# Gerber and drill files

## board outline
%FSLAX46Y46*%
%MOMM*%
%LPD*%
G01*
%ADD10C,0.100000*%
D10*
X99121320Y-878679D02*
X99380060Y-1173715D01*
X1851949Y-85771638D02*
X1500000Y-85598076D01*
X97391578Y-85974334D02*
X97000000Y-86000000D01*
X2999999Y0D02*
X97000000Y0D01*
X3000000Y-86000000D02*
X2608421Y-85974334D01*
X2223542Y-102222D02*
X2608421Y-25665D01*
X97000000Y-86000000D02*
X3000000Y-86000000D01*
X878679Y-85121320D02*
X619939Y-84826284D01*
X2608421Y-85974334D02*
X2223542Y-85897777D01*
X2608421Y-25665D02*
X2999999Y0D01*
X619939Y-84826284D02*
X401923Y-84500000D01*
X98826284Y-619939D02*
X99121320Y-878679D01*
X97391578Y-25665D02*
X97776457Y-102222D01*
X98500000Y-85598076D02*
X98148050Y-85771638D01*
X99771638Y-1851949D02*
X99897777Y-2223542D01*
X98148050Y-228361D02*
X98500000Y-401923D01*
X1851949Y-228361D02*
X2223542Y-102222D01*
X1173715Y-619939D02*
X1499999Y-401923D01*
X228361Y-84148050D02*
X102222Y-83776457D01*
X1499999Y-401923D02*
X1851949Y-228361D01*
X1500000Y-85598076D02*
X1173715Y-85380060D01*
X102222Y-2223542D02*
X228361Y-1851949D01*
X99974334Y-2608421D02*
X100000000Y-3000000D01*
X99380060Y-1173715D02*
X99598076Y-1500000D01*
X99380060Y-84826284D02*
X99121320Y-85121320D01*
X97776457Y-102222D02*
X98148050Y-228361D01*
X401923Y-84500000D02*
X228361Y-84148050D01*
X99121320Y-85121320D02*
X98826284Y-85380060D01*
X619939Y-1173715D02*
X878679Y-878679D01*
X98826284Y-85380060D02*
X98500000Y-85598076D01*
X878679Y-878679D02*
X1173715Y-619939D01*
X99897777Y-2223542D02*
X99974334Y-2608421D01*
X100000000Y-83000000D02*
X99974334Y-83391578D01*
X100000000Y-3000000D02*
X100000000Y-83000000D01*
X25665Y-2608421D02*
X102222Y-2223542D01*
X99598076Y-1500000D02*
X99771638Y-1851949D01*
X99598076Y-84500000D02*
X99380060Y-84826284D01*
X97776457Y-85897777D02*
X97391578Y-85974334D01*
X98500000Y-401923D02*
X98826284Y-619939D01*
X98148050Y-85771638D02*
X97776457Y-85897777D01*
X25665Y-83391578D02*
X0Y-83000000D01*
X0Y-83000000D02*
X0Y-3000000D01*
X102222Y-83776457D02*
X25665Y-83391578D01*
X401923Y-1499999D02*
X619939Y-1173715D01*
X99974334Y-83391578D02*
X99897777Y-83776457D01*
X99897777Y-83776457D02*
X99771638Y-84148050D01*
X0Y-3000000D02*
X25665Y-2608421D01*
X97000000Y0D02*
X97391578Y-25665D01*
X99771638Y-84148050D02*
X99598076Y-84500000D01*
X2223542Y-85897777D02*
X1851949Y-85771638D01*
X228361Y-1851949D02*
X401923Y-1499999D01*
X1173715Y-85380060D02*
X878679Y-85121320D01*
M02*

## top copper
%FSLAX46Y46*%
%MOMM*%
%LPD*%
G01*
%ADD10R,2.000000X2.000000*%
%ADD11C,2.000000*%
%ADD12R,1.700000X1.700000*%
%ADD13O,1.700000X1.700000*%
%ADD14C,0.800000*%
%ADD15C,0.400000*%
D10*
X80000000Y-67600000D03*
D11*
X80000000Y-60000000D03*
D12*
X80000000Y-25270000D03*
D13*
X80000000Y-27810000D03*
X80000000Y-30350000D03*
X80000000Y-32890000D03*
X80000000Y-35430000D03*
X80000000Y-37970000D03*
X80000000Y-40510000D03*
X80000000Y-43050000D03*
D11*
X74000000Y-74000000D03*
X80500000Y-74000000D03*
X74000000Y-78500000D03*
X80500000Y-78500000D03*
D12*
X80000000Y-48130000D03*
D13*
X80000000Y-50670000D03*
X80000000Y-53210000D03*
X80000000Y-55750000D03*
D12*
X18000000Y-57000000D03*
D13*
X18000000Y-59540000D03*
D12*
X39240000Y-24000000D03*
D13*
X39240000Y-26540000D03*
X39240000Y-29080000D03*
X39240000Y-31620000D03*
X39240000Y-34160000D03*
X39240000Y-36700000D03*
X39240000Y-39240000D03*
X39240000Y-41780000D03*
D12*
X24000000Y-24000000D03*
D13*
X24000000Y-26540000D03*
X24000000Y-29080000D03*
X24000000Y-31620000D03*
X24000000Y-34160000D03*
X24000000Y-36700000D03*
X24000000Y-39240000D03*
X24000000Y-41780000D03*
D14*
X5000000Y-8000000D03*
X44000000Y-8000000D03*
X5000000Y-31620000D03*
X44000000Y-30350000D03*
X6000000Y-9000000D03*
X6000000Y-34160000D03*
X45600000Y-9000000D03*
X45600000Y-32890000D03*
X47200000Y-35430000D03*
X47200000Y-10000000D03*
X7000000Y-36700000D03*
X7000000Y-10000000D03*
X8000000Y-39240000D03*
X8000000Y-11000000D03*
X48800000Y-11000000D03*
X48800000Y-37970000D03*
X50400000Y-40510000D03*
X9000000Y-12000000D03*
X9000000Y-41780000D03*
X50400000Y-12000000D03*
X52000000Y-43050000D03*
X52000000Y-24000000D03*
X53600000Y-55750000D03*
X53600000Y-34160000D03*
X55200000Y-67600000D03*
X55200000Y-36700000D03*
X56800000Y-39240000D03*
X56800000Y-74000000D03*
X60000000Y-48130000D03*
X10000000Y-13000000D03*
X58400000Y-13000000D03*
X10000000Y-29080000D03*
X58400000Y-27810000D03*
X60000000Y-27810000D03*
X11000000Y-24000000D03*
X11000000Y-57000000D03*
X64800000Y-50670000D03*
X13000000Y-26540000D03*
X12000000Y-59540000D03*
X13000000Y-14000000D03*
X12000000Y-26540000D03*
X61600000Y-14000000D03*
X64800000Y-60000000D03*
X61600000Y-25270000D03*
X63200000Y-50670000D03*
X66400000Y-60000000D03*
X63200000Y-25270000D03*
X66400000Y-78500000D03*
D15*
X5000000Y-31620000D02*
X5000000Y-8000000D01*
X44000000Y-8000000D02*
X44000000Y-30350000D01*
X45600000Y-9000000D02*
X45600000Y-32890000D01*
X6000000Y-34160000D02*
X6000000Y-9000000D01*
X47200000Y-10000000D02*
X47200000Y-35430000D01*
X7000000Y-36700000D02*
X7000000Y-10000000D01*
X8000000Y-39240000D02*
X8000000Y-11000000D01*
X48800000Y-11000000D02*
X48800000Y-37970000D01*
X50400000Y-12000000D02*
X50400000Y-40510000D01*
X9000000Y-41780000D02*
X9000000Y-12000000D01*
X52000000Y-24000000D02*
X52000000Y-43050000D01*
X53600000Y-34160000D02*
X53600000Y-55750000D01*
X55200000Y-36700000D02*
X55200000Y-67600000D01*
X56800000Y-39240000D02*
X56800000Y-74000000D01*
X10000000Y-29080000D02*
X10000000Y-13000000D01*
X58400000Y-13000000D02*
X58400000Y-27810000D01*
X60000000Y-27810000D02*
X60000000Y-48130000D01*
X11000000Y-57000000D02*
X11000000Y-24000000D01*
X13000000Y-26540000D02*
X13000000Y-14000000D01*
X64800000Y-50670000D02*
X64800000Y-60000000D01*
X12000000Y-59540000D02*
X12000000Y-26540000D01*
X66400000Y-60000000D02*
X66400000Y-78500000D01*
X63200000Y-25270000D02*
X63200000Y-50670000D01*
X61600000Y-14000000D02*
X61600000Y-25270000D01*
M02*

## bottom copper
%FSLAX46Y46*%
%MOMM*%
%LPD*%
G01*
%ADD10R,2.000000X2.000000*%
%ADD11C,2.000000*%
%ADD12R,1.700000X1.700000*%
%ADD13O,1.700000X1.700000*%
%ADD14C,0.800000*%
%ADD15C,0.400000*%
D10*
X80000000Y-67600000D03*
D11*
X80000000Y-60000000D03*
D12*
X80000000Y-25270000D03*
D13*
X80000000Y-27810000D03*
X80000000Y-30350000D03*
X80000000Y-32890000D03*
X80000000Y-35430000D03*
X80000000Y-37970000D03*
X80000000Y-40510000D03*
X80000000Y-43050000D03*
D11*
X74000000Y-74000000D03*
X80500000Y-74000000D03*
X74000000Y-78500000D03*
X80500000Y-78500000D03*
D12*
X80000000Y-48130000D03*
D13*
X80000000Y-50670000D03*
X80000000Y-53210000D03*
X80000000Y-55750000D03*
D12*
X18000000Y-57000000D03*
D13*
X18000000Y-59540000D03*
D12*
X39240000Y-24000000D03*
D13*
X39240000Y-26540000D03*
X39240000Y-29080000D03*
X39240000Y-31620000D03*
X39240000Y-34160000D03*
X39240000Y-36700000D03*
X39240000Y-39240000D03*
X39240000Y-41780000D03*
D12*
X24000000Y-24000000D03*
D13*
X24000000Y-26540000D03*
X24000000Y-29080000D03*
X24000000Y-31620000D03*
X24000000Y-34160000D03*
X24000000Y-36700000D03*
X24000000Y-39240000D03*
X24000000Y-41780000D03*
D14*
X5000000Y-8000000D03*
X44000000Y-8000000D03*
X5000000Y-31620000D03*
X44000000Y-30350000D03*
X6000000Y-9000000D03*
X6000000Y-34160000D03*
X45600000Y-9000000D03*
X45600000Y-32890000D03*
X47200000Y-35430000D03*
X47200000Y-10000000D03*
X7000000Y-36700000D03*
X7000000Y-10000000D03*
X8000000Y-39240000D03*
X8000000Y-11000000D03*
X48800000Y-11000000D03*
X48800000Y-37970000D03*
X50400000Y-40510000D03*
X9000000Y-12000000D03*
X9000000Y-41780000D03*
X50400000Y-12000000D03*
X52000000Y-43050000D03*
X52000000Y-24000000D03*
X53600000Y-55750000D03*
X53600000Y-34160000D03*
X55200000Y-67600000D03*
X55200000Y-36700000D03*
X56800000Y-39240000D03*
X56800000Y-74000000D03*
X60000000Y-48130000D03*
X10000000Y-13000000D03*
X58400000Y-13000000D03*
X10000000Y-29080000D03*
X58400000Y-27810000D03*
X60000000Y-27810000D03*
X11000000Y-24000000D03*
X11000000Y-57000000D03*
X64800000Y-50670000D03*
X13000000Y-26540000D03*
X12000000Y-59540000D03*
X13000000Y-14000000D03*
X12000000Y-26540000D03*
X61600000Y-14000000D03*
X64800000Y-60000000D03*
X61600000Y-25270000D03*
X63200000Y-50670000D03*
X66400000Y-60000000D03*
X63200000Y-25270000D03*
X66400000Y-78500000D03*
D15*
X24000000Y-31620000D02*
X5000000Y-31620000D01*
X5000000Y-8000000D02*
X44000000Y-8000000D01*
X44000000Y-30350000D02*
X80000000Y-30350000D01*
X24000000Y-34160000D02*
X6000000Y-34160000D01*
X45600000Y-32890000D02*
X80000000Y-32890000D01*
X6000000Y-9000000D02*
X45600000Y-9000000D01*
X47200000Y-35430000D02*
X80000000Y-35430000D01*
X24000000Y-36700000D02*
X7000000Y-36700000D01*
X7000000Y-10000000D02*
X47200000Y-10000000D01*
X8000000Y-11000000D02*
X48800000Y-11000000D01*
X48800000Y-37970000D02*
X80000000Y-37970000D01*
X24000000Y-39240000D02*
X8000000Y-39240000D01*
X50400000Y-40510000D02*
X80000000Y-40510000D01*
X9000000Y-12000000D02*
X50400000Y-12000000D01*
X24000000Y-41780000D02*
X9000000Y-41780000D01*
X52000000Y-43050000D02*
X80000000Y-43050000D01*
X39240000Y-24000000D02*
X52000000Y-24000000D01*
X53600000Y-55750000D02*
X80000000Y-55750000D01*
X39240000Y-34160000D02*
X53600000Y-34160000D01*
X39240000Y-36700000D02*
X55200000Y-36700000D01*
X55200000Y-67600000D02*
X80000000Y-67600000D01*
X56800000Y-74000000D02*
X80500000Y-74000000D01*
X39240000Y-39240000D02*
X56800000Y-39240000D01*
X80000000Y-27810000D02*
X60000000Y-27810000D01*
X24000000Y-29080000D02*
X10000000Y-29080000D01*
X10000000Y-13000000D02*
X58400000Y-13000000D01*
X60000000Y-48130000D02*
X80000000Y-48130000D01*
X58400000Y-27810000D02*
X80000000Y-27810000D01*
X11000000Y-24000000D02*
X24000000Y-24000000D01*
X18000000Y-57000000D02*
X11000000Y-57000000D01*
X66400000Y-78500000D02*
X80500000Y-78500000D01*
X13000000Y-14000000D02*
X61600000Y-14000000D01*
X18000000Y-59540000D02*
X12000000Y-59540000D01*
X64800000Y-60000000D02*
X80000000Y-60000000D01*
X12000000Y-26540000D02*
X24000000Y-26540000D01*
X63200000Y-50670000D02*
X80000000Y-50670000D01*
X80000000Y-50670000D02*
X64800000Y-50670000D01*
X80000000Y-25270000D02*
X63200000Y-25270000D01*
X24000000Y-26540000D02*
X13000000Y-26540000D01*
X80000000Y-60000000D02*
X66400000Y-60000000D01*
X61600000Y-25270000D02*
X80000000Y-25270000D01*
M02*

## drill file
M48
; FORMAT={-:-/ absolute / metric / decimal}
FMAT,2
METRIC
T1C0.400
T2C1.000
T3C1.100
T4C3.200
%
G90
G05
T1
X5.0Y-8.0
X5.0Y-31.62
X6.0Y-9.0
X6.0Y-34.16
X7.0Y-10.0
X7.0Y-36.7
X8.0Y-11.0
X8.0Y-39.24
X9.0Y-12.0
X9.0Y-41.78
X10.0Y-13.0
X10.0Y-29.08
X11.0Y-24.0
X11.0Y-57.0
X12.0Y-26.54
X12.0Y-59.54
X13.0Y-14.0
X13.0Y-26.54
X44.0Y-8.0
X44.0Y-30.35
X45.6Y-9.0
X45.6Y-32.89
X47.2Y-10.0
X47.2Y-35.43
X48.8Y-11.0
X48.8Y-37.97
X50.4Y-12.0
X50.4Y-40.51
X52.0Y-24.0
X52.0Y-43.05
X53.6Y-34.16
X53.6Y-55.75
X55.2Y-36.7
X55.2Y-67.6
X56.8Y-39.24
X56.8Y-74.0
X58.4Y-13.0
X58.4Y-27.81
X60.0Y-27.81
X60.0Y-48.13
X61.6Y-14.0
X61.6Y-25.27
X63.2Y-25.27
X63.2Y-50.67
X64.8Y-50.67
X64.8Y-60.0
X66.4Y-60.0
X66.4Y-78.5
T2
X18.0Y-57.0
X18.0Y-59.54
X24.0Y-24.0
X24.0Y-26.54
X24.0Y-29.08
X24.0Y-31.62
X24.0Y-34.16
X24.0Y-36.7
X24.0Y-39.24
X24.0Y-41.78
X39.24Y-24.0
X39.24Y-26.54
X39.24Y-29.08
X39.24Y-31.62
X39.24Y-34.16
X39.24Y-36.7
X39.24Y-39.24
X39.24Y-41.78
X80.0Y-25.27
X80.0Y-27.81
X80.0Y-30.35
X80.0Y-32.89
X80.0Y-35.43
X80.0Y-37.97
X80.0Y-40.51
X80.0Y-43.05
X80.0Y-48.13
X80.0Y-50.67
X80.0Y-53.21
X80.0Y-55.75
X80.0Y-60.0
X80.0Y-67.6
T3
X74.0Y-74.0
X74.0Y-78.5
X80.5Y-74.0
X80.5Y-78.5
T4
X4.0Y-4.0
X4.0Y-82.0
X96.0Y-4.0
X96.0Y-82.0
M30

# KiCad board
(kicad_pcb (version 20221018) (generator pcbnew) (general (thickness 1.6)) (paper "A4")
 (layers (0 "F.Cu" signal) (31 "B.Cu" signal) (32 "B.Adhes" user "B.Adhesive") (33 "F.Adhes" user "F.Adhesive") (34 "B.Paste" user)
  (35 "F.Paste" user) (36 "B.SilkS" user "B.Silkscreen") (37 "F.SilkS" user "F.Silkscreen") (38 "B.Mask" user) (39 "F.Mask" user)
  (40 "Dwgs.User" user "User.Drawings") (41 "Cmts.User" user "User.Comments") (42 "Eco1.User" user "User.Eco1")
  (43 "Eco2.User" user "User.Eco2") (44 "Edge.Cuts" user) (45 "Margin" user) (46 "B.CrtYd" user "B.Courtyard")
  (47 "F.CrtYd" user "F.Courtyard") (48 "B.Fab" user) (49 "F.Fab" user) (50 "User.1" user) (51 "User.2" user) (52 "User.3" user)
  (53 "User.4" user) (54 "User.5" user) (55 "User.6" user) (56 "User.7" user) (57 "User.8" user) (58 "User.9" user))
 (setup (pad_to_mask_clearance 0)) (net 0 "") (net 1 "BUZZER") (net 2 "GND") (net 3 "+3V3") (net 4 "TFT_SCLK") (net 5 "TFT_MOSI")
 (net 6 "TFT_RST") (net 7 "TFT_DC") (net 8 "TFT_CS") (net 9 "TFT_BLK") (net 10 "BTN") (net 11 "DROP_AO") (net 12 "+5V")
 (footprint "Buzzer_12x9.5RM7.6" (layer "F.Cu") (at 80 67.6 90)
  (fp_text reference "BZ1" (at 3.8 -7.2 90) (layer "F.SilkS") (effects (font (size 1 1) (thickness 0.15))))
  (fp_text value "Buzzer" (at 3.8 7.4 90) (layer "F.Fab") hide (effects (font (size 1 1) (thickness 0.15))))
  (pad "1" thru_hole rect (at 0 0 90) (size 2 2) (drill 1) (layers "*.Cu" "*.Mask") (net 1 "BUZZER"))
  (pad "2" thru_hole circle (at 7.6 0 90) (size 2 2) (drill 1) (layers "*.Cu" "*.Mask") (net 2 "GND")))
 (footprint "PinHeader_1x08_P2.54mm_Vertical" (layer "F.Cu") (at 80 25.27)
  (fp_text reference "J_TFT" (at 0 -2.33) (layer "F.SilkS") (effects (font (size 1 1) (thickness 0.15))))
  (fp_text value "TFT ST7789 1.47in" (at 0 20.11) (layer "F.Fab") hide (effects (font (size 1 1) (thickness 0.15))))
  (pad "1" thru_hole rect (at 0 0) (size 1.7 1.7) (drill 1) (layers "*.Cu" "*.Mask") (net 2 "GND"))
  (pad "2" thru_hole oval (at 0 2.54) (size 1.7 1.7) (drill 1) (layers "*.Cu" "*.Mask") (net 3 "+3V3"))
  (pad "3" thru_hole oval (at 0 5.08) (size 1.7 1.7) (drill 1) (layers "*.Cu" "*.Mask") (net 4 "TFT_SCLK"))
  (pad "4" thru_hole oval (at 0 7.62) (size 1.7 1.7) (drill 1) (layers "*.Cu" "*.Mask") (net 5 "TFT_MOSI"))
  (pad "5" thru_hole oval (at 0 10.16) (size 1.7 1.7) (drill 1) (layers "*.Cu" "*.Mask") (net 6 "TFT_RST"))
  (pad "6" thru_hole oval (at 0 12.7) (size 1.7 1.7) (drill 1) (layers "*.Cu" "*.Mask") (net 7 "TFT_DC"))
  (pad "7" thru_hole oval (at 0 15.24) (size 1.7 1.7) (drill 1) (layers "*.Cu" "*.Mask") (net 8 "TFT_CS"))
  (pad "8" thru_hole oval (at 0 17.78) (size 1.7 1.7) (drill 1) (layers "*.Cu" "*.Mask") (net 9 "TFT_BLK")))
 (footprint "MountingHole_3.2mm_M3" (layer "F.Cu") (at 4 4)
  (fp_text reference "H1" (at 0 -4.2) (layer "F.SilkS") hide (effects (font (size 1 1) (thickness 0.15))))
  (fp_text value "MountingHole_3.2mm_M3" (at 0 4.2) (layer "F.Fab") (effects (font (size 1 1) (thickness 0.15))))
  (pad "" np_thru_hole circle (at 0 0) (size 3.2 3.2) (drill 3.2) (layers "*.Cu" "*.Mask")))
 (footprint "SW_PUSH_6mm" (layer "F.Cu") (at 74 74)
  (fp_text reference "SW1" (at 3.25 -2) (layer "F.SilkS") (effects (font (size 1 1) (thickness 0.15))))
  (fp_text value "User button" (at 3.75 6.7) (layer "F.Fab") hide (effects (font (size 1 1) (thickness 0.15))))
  (pad "1" thru_hole circle (at 0 0 90) (size 2 2) (drill 1.1) (layers "*.Cu" "*.Mask") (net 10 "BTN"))
  (pad "1" thru_hole circle (at 6.5 0 90) (size 2 2) (drill 1.1) (layers "*.Cu" "*.Mask") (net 10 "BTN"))
  (pad "2" thru_hole circle (at 0 4.5 90) (size 2 2) (drill 1.1) (layers "*.Cu" "*.Mask") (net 2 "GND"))
  (pad "2" thru_hole circle (at 6.5 4.5 90) (size 2 2) (drill 1.1) (layers "*.Cu" "*.Mask") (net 2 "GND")))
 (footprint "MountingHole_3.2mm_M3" (layer "F.Cu") (at 96 82)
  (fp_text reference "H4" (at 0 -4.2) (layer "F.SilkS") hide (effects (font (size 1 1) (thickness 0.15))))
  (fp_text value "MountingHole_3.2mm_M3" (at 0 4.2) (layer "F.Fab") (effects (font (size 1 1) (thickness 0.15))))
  (pad "" np_thru_hole circle (at 0 0) (size 3.2 3.2) (drill 3.2) (layers "*.Cu" "*.Mask")))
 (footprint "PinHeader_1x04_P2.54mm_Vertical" (layer "F.Cu") (at 80 48.13)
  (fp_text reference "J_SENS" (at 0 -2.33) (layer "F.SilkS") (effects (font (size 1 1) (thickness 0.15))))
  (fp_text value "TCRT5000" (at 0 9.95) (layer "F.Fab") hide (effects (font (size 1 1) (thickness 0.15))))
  (pad "1" thru_hole rect (at 0 0) (size 1.7 1.7) (drill 1) (layers "*.Cu" "*.Mask") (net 3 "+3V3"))
  (pad "2" thru_hole oval (at 0 2.54) (size 1.7 1.7) (drill 1) (layers "*.Cu" "*.Mask") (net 2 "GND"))
  (pad "3" thru_hole oval (at 0 5.08) (size 1.7 1.7) (drill 1) (layers "*.Cu" "*.Mask"))
  (pad "4" thru_hole oval (at 0 7.62) (size 1.7 1.7) (drill 1) (layers "*.Cu" "*.Mask") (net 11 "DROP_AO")))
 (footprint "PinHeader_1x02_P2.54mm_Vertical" (layer "F.Cu") (at 18 57)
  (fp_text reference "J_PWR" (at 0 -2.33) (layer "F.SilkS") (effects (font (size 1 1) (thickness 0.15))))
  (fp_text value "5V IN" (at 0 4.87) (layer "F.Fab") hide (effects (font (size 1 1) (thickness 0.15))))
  (pad "1" thru_hole rect (at 0 0) (size 1.7 1.7) (drill 1) (layers "*.Cu" "*.Mask") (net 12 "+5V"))
  (pad "2" thru_hole oval (at 0 2.54) (size 1.7 1.7) (drill 1) (layers "*.Cu" "*.Mask") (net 2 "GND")))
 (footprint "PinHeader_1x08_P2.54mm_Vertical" (layer "F.Cu") (at 39.24 24)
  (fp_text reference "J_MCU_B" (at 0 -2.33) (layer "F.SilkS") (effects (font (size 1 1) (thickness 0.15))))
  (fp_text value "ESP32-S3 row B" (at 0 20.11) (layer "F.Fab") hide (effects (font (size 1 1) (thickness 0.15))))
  (pad "1" thru_hole rect (at 0 0) (size 1.7 1.7) (drill 1) (layers "*.Cu" "*.Mask") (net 9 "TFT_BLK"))
  (pad "2" thru_hole oval (at 0 2.54) (size 1.7 1.7) (drill 1) (layers "*.Cu" "*.Mask"))
  (pad "3" thru_hole oval (at 0 5.08) (size 1.7 1.7) (drill 1) (layers "*.Cu" "*.Mask"))
  (pad "4" thru_hole oval (at 0 7.62) (size 1.7 1.7) (drill 1) (layers "*.Cu" "*.Mask"))
  (pad "5" thru_hole oval (at 0 10.16) (size 1.7 1.7) (drill 1) (layers "*.Cu" "*.Mask") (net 11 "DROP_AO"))
  (pad "6" thru_hole oval (at 0 12.7) (size 1.7 1.7) (drill 1) (layers "*.Cu" "*.Mask") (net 1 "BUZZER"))
  (pad "7" thru_hole oval (at 0 15.24) (size 1.7 1.7) (drill 1) (layers "*.Cu" "*.Mask") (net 10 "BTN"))
  (pad "8" thru_hole oval (at 0 17.78) (size 1.7 1.7) (drill 1) (layers "*.Cu" "*.Mask")))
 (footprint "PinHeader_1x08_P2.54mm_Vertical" (layer "F.Cu") (at 24 24)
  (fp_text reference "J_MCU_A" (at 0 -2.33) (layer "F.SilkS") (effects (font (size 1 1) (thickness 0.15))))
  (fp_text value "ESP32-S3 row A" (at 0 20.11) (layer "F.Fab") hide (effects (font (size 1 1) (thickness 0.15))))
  (pad "1" thru_hole rect (at 0 0) (size 1.7 1.7) (drill 1) (layers "*.Cu" "*.Mask") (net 12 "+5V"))
  (pad "2" thru_hole oval (at 0 2.54) (size 1.7 1.7) (drill 1) (layers "*.Cu" "*.Mask") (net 2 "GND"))
  (pad "3" thru_hole oval (at 0 5.08) (size 1.7 1.7) (drill 1) (layers "*.Cu" "*.Mask") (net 3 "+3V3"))
  (pad "4" thru_hole oval (at 0 7.62) (size 1.7 1.7) (drill 1) (layers "*.Cu" "*.Mask") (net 4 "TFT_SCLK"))
  (pad "5" thru_hole oval (at 0 10.16) (size 1.7 1.7) (drill 1) (layers "*.Cu" "*.Mask") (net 5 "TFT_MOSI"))
  (pad "6" thru_hole oval (at 0 12.7) (size 1.7 1.7) (drill 1) (layers "*.Cu" "*.Mask") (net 6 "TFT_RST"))
  (pad "7" thru_hole oval (at 0 15.24) (size 1.7 1.7) (drill 1) (layers "*.Cu" "*.Mask") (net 7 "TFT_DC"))
  (pad "8" thru_hole oval (at 0 17.78) (size 1.7 1.7) (drill 1) (layers "*.Cu" "*.Mask") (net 8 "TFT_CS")))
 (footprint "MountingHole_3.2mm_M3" (layer "F.Cu") (at 4 82)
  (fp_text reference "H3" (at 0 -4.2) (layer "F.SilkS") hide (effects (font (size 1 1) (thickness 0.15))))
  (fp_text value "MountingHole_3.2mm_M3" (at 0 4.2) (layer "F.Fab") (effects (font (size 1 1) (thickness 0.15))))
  (pad "" np_thru_hole circle (at 0 0) (size 3.2 3.2) (drill 3.2) (layers "*.Cu" "*.Mask")))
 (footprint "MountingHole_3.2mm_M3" (layer "F.Cu") (at 96 4)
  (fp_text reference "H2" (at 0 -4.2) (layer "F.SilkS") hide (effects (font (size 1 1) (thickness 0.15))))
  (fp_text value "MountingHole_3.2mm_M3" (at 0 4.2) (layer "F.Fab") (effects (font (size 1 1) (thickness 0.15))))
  (pad "" np_thru_hole circle (at 0 0) (size 3.2 3.2) (drill 3.2) (layers "*.Cu" "*.Mask")))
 (gr_line (start 99.12132 0.878679) (end 99.38006 1.173715) (stroke (width 0.1) (type default)) (layer "Edge.Cuts"))
 (gr_line (start 1.851949 85.771638) (end 1.5 85.598076) (stroke (width 0.1) (type default)) (layer "Edge.Cuts"))
 (gr_line (start 97.391578 85.974334) (end 97 86) (stroke (width 0.1) (type default)) (layer "Edge.Cuts"))
 (gr_line (start 2.999999 0) (end 97 0) (stroke (width 0.1) (type default)) (layer "Edge.Cuts"))
 (gr_line (start 3 86) (end 2.608421 85.974334) (stroke (width 0.1) (type default)) (layer "Edge.Cuts"))
 (gr_line (start 2.223542 0.102222) (end 2.608421 0.025665) (stroke (width 0.1) (type default)) (layer "Edge.Cuts"))
 (gr_line (start 97 86) (end 3 86) (stroke (width 0.1) (type default)) (layer "Edge.Cuts"))
 (gr_line (start 0.878679 85.12132) (end 0.619939 84.826284) (stroke (width 0.1) (type default)) (layer "Edge.Cuts"))
 (gr_line (start 2.608421 85.974334) (end 2.223542 85.897777) (stroke (width 0.1) (type default)) (layer "Edge.Cuts"))
 (gr_line (start 2.608421 0.025665) (end 2.999999 0) (stroke (width 0.1) (type default)) (layer "Edge.Cuts"))
 (gr_line (start 0.619939 84.826284) (end 0.401923 84.5) (stroke (width 0.1) (type default)) (layer "Edge.Cuts"))
 (gr_line (start 98.826284 0.619939) (end 99.12132 0.878679) (stroke (width 0.1) (type default)) (layer "Edge.Cuts"))
 (gr_line (start 97.391578 0.025665) (end 97.776457 0.102222) (stroke (width 0.1) (type default)) (layer "Edge.Cuts"))
 (gr_line (start 98.5 85.598076) (end 98.14805 85.771638) (stroke (width 0.1) (type default)) (layer "Edge.Cuts"))
 (gr_line (start 99.771638 1.851949) (end 99.897777 2.223542) (stroke (width 0.1) (type default)) (layer "Edge.Cuts"))
 (gr_line (start 98.14805 0.228361) (end 98.5 0.401923) (stroke (width 0.1) (type default)) (layer "Edge.Cuts"))
 (gr_line (start 1.851949 0.228361) (end 2.223542 0.102222) (stroke (width 0.1) (type default)) (layer "Edge.Cuts"))
 (gr_line (start 1.173715 0.619939) (end 1.499999 0.401923) (stroke (width 0.1) (type default)) (layer "Edge.Cuts"))
 (gr_line (start 0.228361 84.14805) (end 0.102222 83.776457) (stroke (width 0.1) (type default)) (layer "Edge.Cuts"))
 (gr_line (start 1.499999 0.401923) (end 1.851949 0.228361) (stroke (width 0.1) (type default)) (layer "Edge.Cuts"))
 (gr_line (start 1.5 85.598076) (end 1.173715 85.38006) (stroke (width 0.1) (type default)) (layer "Edge.Cuts"))
 (gr_line (start 0.102222 2.223542) (end 0.228361 1.851949) (stroke (width 0.1) (type default)) (layer "Edge.Cuts"))
 (gr_line (start 99.974334 2.608421) (end 100 3) (stroke (width 0.1) (type default)) (layer "Edge.Cuts"))
 (gr_line (start 99.38006 1.173715) (end 99.598076 1.5) (stroke (width 0.1) (type default)) (layer "Edge.Cuts"))
 (gr_line (start 99.38006 84.826284) (end 99.12132 85.12132) (stroke (width 0.1) (type default)) (layer "Edge.Cuts"))
 (gr_line (start 97.776457 0.102222) (end 98.14805 0.228361) (stroke (width 0.1) (type default)) (layer "Edge.Cuts"))
 (gr_line (start 0.401923 84.5) (end 0.228361 84.14805) (stroke (width 0.1) (type default)) (layer "Edge.Cuts"))
 (gr_line (start 99.12132 85.12132) (end 98.826284 85.38006) (stroke (width 0.1) (type default)) (layer "Edge.Cuts"))
 (gr_line (start 0.619939 1.173715) (end 0.878679 0.878679) (stroke (width 0.1) (type default)) (layer "Edge.Cuts"))
 (gr_line (start 98.826284 85.38006) (end 98.5 85.598076) (stroke (width 0.1) (type default)) (layer "Edge.Cuts"))
 (gr_line (start 0.878679 0.878679) (end 1.173715 0.619939) (stroke (width 0.1) (type default)) (layer "Edge.Cuts"))
 (gr_line (start 99.897777 2.223542) (end 99.974334 2.608421) (stroke (width 0.1) (type default)) (layer "Edge.Cuts"))
 (gr_line (start 100 83) (end 99.974334 83.391578) (stroke (width 0.1) (type default)) (layer "Edge.Cuts"))
 (gr_line (start 100 3) (end 100 83) (stroke (width 0.1) (type default)) (layer "Edge.Cuts"))
 (gr_line (start 0.025665 2.608421) (end 0.102222 2.223542) (stroke (width 0.1) (type default)) (layer "Edge.Cuts"))
 (gr_line (start 99.598076 1.5) (end 99.771638 1.851949) (stroke (width 0.1) (type default)) (layer "Edge.Cuts"))
 (gr_line (start 99.598076 84.5) (end 99.38006 84.826284) (stroke (width 0.1) (type default)) (layer "Edge.Cuts"))
 (gr_line (start 97.776457 85.897777) (end 97.391578 85.974334) (stroke (width 0.1) (type default)) (layer "Edge.Cuts"))
 (gr_line (start 98.5 0.401923) (end 98.826284 0.619939) (stroke (width 0.1) (type default)) (layer "Edge.Cuts"))
 (gr_line (start 98.14805 85.771638) (end 97.776457 85.897777) (stroke (width 0.1) (type default)) (layer "Edge.Cuts"))
 (gr_line (start 0.025665 83.391578) (end 0 83) (stroke (width 0.1) (type default)) (layer "Edge.Cuts"))
 (gr_line (start 0 83) (end 0 3) (stroke (width 0.1) (type default)) (layer "Edge.Cuts"))
 (gr_line (start 0.102222 83.776457) (end 0.025665 83.391578) (stroke (width 0.1) (type default)) (layer "Edge.Cuts"))
 (gr_line (start 0.401923 1.499999) (end 0.619939 1.173715) (stroke (width 0.1) (type default)) (layer "Edge.Cuts"))
 (gr_line (start 99.974334 83.391578) (end 99.897777 83.776457) (stroke (width 0.1) (type default)) (layer "Edge.Cuts"))
 (gr_line (start 99.897777 83.776457) (end 99.771638 84.14805) (stroke (width 0.1) (type default)) (layer "Edge.Cuts"))
 (gr_line (start 0 3) (end 0.025665 2.608421) (stroke (width 0.1) (type default)) (layer "Edge.Cuts"))
 (gr_line (start 97 0) (end 97.391578 0.025665) (stroke (width 0.1) (type default)) (layer "Edge.Cuts"))
 (gr_line (start 99.771638 84.14805) (end 99.598076 84.5) (stroke (width 0.1) (type default)) (layer "Edge.Cuts"))
 (gr_line (start 2.223542 85.897777) (end 1.851949 85.771638) (stroke (width 0.1) (type default)) (layer "Edge.Cuts"))
 (gr_line (start 0.228361 1.851949) (end 0.401923 1.499999) (stroke (width 0.1) (type default)) (layer "Edge.Cuts"))
 (gr_line (start 1.173715 85.38006) (end 0.878679 85.12132) (stroke (width 0.1) (type default)) (layer "Edge.Cuts"))
 (segment (start 5 31.62) (end 5 8) (width 0.4) (layer "F.Cu") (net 4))
 (segment (start 44 8) (end 44 30.35) (width 0.4) (layer "F.Cu") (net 4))
 (via (at 5 8) (size 0.8) (drill 0.4) (layers "F.Cu" "B.Cu") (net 4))
 (via (at 44 8) (size 0.8) (drill 0.4) (layers "F.Cu" "B.Cu") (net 4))
 (via (at 5 31.62) (size 0.8) (drill 0.4) (layers "F.Cu" "B.Cu") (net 4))
 (via (at 44 30.35) (size 0.8) (drill 0.4) (layers "F.Cu" "B.Cu") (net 4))
 (segment (start 24 31.62) (end 5 31.62) (width 0.4) (layer "B.Cu") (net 4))
 (segment (start 5 8) (end 44 8) (width 0.4) (layer "B.Cu") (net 4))
 (segment (start 44 30.35) (end 80 30.35) (width 0.4) (layer "B.Cu") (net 4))
 (segment (start 45.6 9) (end 45.6 32.89) (width 0.4) (layer "F.Cu") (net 5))
 (segment (start 6 34.16) (end 6 9) (width 0.4) (layer "F.Cu") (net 5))
 (via (at 6 9) (size 0.8) (drill 0.4) (layers "F.Cu" "B.Cu") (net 5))
 (via (at 6 34.16) (size 0.8) (drill 0.4) (layers "F.Cu" "B.Cu") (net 5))
 (via (at 45.6 9) (size 0.8) (drill 0.4) (layers "F.Cu" "B.Cu") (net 5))
 (via (at 45.6 32.89) (size 0.8) (drill 0.4) (layers "F.Cu" "B.Cu") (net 5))
 (segment (start 24 34.16) (end 6 34.16) (width 0.4) (layer "B.Cu") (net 5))
 (segment (start 45.6 32.89) (end 80 32.89) (width 0.4) (layer "B.Cu") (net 5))
 (segment (start 6 9) (end 45.6 9) (width 0.4) (layer "B.Cu") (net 5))
 (segment (start 47.2 10) (end 47.2 35.43) (width 0.4) (layer "F.Cu") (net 6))
 (segment (start 7 36.7) (end 7 10) (width 0.4) (layer "F.Cu") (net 6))
 (via (at 47.2 35.43) (size 0.8) (drill 0.4) (layers "F.Cu" "B.Cu") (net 6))
 (via (at 47.2 10) (size 0.8) (drill 0.4) (layers "F.Cu" "B.Cu") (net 6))
 (via (at 7 36.7) (size 0.8) (drill 0.4) (layers "F.Cu" "B.Cu") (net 6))
 (via (at 7 10) (size 0.8) (drill 0.4) (layers "F.Cu" "B.Cu") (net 6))
 (segment (start 47.2 35.43) (end 80 35.43) (width 0.4) (layer "B.Cu") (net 6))
 (segment (start 24 36.7) (end 7 36.7) (width 0.4) (layer "B.Cu") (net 6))
 (segment (start 7 10) (end 47.2 10) (width 0.4) (layer "B.Cu") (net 6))
 (segment (start 8 39.24) (end 8 11) (width 0.4) (layer "F.Cu") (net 7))
 (segment (start 48.8 11) (end 48.8 37.97) (width 0.4) (layer "F.Cu") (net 7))
 (via (at 8 39.24) (size 0.8) (drill 0.4) (layers "F.Cu" "B.Cu") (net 7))
 (via (at 8 11) (size 0.8) (drill 0.4) (layers "F.Cu" "B.Cu") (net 7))
 (via (at 48.8 11) (size 0.8) (drill 0.4) (layers "F.Cu" "B.Cu") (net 7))
 (via (at 48.8 37.97) (size 0.8) (drill 0.4) (layers "F.Cu" "B.Cu") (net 7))
 (segment (start 8 11) (end 48.8 11) (width 0.4) (layer "B.Cu") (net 7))
 (segment (start 48.8 37.97) (end 80 37.97) (width 0.4) (layer "B.Cu") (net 7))
 (segment (start 24 39.24) (end 8 39.24) (width 0.4) (layer "B.Cu") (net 7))
 (segment (start 50.4 12) (end 50.4 40.51) (width 0.4) (layer "F.Cu") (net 8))
 (segment (start 9 41.78) (end 9 12) (width 0.4) (layer "F.Cu") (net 8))
 (via (at 50.4 40.51) (size 0.8) (drill 0.4) (layers "F.Cu" "B.Cu") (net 8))
 (via (at 9 12) (size 0.8) (drill 0.4) (layers "F.Cu" "B.Cu") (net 8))
 (via (at 9 41.78) (size 0.8) (drill 0.4) (layers "F.Cu" "B.Cu") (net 8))
 (via (at 50.4 12) (size 0.8) (drill 0.4) (layers "F.Cu" "B.Cu") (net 8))
 (segment (start 50.4 40.51) (end 80 40.51) (width 0.4) (layer "B.Cu") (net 8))
 (segment (start 9 12) (end 50.4 12) (width 0.4) (layer "B.Cu") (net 8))
 (segment (start 24 41.78) (end 9 41.78) (width 0.4) (layer "B.Cu") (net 8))
 (segment (start 52 24) (end 52 43.05) (width 0.4) (layer "F.Cu") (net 9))
 (via (at 52 43.05) (size 0.8) (drill 0.4) (layers "F.Cu" "B.Cu") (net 9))
 (via (at 52 24) (size 0.8) (drill 0.4) (layers "F.Cu" "B.Cu") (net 9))
 (segment (start 52 43.05) (end 80 43.05) (width 0.4) (layer "B.Cu") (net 9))
 (segment (start 39.24 24) (end 52 24) (width 0.4) (layer "B.Cu") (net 9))
 (segment (start 53.6 34.16) (end 53.6 55.75) (width 0.4) (layer "F.Cu") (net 11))
 (via (at 53.6 55.75) (size 0.8) (drill 0.4) (layers "F.Cu" "B.Cu") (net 11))
 (via (at 53.6 34.16) (size 0.8) (drill 0.4) (layers "F.Cu" "B.Cu") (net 11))
 (segment (start 53.6 55.75) (end 80 55.75) (width 0.4) (layer "B.Cu") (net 11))
 (segment (start 39.24 34.16) (end 53.6 34.16) (width 0.4) (layer "B.Cu") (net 11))
 (segment (start 55.2 36.7) (end 55.2 67.6) (width 0.4) (layer "F.Cu") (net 1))
 (via (at 55.2 67.6) (size 0.8) (drill 0.4) (layers "F.Cu" "B.Cu") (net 1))
 (via (at 55.2 36.7) (size 0.8) (drill 0.4) (layers "F.Cu" "B.Cu") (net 1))
 (segment (start 39.24 36.7) (end 55.2 36.7) (width 0.4) (layer "B.Cu") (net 1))
 (segment (start 55.2 67.6) (end 80 67.6) (width 0.4) (layer "B.Cu") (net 1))
 (segment (start 56.8 39.24) (end 56.8 74) (width 0.4) (layer "F.Cu") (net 10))
 (via (at 56.8 39.24) (size 0.8) (drill 0.4) (layers "F.Cu" "B.Cu") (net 10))
 (via (at 56.8 74) (size 0.8) (drill 0.4) (layers "F.Cu" "B.Cu") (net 10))
 (segment (start 56.8 74) (end 80.5 74) (width 0.4) (layer "B.Cu") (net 10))
 (segment (start 39.24 39.24) (end 56.8 39.24) (width 0.4) (layer "B.Cu") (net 10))
 (segment (start 10 29.08) (end 10 13) (width 0.4) (layer "F.Cu") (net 3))
 (segment (start 58.4 13) (end 58.4 27.81) (width 0.4) (layer "F.Cu") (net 3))
 (segment (start 60 27.81) (end 60 48.13) (width 0.4) (layer "F.Cu") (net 3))
 (via (at 60 48.13) (size 0.8) (drill 0.4) (layers "F.Cu" "B.Cu") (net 3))
 (via (at 10 13) (size 0.8) (drill 0.4) (layers "F.Cu" "B.Cu") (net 3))
 (via (at 58.4 13) (size 0.8) (drill 0.4) (layers "F.Cu" "B.Cu") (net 3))
 (via (at 10 29.08) (size 0.8) (drill 0.4) (layers "F.Cu" "B.Cu") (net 3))
 (via (at 58.4 27.81) (size 0.8) (drill 0.4) (layers "F.Cu" "B.Cu") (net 3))
 (via (at 60 27.81) (size 0.8) (drill 0.4) (layers "F.Cu" "B.Cu") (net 3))
 (segment (start 80 27.81) (end 60 27.81) (width 0.4) (layer "B.Cu") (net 3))
 (segment (start 24 29.08) (end 10 29.08) (width 0.4) (layer "B.Cu") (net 3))
 (segment (start 10 13) (end 58.4 13) (width 0.4) (layer "B.Cu") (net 3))
 (segment (start 60 48.13) (end 80 48.13) (width 0.4) (layer "B.Cu") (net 3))
 (segment (start 58.4 27.81) (end 80 27.81) (width 0.4) (layer "B.Cu") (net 3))
 (segment (start 11 57) (end 11 24) (width 0.4) (layer "F.Cu") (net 12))
 (via (at 11 24) (size 0.8) (drill 0.4) (layers "F.Cu" "B.Cu") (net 12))
 (via (at 11 57) (size 0.8) (drill 0.4) (layers "F.Cu" "B.Cu") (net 12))
 (segment (start 11 24) (end 24 24) (width 0.4) (layer "B.Cu") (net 12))
 (segment (start 18 57) (end 11 57) (width 0.4) (layer "B.Cu") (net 12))
 (segment (start 13 26.54) (end 13 14) (width 0.4) (layer "F.Cu") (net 2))
 (segment (start 64.8 50.67) (end 64.8 60) (width 0.4) (layer "F.Cu") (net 2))
 (segment (start 12 59.54) (end 12 26.54) (width 0.4) (layer "F.Cu") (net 2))
 (segment (start 66.4 60) (end 66.4 78.5) (width 0.4) (layer "F.Cu") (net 2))
 (segment (start 63.2 25.27) (end 63.2 50.67) (width 0.4) (layer "F.Cu") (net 2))
 (segment (start 61.6 14) (end 61.6 25.27) (width 0.4) (layer "F.Cu") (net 2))
 (via (at 64.8 50.67) (size 0.8) (drill 0.4) (layers "F.Cu" "B.Cu") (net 2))
 (via (at 13 26.54) (size 0.8) (drill 0.4) (layers "F.Cu" "B.Cu") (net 2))
 (via (at 12 59.54) (size 0.8) (drill 0.4) (layers "F.Cu" "B.Cu") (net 2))
 (via (at 13 14) (size 0.8) (drill 0.4) (layers "F.Cu" "B.Cu") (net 2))
 (via (at 12 26.54) (size 0.8) (drill 0.4) (layers "F.Cu" "B.Cu") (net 2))
 (via (at 61.6 14) (size 0.8) (drill 0.4) (layers "F.Cu" "B.Cu") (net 2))
 (via (at 64.8 60) (size 0.8) (drill 0.4) (layers "F.Cu" "B.Cu") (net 2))
 (via (at 61.6 25.27) (size 0.8) (drill 0.4) (layers "F.Cu" "B.Cu") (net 2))
 (via (at 63.2 50.67) (size 0.8) (drill 0.4) (layers "F.Cu" "B.Cu") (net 2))
 (via (at 66.4 60) (size 0.8) (drill 0.4) (layers "F.Cu" "B.Cu") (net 2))
 (via (at 63.2 25.27) (size 0.8) (drill 0.4) (layers "F.Cu" "B.Cu") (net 2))
 (via (at 66.4 78.5) (size 0.8) (drill 0.4) (layers "F.Cu" "B.Cu") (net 2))
 (segment (start 66.4 78.5) (end 80.5 78.5) (width 0.4) (layer "B.Cu") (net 2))
 (segment (start 13 14) (end 61.6 14) (width 0.4) (layer "B.Cu") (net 2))
 (segment (start 18 59.54) (end 12 59.54) (width 0.4) (layer "B.Cu") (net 2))
 (segment (start 64.8 60) (end 80 60) (width 0.4) (layer "B.Cu") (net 2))
 (segment (start 12 26.54) (end 24 26.54) (width 0.4) (layer "B.Cu") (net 2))
 (segment (start 63.2 50.67) (end 80 50.67) (width 0.4) (layer "B.Cu") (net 2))
 (segment (start 80 50.67) (end 64.8 50.67) (width 0.4) (layer "B.Cu") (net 2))
 (segment (start 80 25.27) (end 63.2 25.27) (width 0.4) (layer "B.Cu") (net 2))
 (segment (start 24 26.54) (end 13 26.54) (width 0.4) (layer "B.Cu") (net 2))
 (segment (start 80 60) (end 66.4 60) (width 0.4) (layer "B.Cu") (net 2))
 (segment (start 61.6 25.27) (end 80 25.27) (width 0.4) (layer "B.Cu") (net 2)))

